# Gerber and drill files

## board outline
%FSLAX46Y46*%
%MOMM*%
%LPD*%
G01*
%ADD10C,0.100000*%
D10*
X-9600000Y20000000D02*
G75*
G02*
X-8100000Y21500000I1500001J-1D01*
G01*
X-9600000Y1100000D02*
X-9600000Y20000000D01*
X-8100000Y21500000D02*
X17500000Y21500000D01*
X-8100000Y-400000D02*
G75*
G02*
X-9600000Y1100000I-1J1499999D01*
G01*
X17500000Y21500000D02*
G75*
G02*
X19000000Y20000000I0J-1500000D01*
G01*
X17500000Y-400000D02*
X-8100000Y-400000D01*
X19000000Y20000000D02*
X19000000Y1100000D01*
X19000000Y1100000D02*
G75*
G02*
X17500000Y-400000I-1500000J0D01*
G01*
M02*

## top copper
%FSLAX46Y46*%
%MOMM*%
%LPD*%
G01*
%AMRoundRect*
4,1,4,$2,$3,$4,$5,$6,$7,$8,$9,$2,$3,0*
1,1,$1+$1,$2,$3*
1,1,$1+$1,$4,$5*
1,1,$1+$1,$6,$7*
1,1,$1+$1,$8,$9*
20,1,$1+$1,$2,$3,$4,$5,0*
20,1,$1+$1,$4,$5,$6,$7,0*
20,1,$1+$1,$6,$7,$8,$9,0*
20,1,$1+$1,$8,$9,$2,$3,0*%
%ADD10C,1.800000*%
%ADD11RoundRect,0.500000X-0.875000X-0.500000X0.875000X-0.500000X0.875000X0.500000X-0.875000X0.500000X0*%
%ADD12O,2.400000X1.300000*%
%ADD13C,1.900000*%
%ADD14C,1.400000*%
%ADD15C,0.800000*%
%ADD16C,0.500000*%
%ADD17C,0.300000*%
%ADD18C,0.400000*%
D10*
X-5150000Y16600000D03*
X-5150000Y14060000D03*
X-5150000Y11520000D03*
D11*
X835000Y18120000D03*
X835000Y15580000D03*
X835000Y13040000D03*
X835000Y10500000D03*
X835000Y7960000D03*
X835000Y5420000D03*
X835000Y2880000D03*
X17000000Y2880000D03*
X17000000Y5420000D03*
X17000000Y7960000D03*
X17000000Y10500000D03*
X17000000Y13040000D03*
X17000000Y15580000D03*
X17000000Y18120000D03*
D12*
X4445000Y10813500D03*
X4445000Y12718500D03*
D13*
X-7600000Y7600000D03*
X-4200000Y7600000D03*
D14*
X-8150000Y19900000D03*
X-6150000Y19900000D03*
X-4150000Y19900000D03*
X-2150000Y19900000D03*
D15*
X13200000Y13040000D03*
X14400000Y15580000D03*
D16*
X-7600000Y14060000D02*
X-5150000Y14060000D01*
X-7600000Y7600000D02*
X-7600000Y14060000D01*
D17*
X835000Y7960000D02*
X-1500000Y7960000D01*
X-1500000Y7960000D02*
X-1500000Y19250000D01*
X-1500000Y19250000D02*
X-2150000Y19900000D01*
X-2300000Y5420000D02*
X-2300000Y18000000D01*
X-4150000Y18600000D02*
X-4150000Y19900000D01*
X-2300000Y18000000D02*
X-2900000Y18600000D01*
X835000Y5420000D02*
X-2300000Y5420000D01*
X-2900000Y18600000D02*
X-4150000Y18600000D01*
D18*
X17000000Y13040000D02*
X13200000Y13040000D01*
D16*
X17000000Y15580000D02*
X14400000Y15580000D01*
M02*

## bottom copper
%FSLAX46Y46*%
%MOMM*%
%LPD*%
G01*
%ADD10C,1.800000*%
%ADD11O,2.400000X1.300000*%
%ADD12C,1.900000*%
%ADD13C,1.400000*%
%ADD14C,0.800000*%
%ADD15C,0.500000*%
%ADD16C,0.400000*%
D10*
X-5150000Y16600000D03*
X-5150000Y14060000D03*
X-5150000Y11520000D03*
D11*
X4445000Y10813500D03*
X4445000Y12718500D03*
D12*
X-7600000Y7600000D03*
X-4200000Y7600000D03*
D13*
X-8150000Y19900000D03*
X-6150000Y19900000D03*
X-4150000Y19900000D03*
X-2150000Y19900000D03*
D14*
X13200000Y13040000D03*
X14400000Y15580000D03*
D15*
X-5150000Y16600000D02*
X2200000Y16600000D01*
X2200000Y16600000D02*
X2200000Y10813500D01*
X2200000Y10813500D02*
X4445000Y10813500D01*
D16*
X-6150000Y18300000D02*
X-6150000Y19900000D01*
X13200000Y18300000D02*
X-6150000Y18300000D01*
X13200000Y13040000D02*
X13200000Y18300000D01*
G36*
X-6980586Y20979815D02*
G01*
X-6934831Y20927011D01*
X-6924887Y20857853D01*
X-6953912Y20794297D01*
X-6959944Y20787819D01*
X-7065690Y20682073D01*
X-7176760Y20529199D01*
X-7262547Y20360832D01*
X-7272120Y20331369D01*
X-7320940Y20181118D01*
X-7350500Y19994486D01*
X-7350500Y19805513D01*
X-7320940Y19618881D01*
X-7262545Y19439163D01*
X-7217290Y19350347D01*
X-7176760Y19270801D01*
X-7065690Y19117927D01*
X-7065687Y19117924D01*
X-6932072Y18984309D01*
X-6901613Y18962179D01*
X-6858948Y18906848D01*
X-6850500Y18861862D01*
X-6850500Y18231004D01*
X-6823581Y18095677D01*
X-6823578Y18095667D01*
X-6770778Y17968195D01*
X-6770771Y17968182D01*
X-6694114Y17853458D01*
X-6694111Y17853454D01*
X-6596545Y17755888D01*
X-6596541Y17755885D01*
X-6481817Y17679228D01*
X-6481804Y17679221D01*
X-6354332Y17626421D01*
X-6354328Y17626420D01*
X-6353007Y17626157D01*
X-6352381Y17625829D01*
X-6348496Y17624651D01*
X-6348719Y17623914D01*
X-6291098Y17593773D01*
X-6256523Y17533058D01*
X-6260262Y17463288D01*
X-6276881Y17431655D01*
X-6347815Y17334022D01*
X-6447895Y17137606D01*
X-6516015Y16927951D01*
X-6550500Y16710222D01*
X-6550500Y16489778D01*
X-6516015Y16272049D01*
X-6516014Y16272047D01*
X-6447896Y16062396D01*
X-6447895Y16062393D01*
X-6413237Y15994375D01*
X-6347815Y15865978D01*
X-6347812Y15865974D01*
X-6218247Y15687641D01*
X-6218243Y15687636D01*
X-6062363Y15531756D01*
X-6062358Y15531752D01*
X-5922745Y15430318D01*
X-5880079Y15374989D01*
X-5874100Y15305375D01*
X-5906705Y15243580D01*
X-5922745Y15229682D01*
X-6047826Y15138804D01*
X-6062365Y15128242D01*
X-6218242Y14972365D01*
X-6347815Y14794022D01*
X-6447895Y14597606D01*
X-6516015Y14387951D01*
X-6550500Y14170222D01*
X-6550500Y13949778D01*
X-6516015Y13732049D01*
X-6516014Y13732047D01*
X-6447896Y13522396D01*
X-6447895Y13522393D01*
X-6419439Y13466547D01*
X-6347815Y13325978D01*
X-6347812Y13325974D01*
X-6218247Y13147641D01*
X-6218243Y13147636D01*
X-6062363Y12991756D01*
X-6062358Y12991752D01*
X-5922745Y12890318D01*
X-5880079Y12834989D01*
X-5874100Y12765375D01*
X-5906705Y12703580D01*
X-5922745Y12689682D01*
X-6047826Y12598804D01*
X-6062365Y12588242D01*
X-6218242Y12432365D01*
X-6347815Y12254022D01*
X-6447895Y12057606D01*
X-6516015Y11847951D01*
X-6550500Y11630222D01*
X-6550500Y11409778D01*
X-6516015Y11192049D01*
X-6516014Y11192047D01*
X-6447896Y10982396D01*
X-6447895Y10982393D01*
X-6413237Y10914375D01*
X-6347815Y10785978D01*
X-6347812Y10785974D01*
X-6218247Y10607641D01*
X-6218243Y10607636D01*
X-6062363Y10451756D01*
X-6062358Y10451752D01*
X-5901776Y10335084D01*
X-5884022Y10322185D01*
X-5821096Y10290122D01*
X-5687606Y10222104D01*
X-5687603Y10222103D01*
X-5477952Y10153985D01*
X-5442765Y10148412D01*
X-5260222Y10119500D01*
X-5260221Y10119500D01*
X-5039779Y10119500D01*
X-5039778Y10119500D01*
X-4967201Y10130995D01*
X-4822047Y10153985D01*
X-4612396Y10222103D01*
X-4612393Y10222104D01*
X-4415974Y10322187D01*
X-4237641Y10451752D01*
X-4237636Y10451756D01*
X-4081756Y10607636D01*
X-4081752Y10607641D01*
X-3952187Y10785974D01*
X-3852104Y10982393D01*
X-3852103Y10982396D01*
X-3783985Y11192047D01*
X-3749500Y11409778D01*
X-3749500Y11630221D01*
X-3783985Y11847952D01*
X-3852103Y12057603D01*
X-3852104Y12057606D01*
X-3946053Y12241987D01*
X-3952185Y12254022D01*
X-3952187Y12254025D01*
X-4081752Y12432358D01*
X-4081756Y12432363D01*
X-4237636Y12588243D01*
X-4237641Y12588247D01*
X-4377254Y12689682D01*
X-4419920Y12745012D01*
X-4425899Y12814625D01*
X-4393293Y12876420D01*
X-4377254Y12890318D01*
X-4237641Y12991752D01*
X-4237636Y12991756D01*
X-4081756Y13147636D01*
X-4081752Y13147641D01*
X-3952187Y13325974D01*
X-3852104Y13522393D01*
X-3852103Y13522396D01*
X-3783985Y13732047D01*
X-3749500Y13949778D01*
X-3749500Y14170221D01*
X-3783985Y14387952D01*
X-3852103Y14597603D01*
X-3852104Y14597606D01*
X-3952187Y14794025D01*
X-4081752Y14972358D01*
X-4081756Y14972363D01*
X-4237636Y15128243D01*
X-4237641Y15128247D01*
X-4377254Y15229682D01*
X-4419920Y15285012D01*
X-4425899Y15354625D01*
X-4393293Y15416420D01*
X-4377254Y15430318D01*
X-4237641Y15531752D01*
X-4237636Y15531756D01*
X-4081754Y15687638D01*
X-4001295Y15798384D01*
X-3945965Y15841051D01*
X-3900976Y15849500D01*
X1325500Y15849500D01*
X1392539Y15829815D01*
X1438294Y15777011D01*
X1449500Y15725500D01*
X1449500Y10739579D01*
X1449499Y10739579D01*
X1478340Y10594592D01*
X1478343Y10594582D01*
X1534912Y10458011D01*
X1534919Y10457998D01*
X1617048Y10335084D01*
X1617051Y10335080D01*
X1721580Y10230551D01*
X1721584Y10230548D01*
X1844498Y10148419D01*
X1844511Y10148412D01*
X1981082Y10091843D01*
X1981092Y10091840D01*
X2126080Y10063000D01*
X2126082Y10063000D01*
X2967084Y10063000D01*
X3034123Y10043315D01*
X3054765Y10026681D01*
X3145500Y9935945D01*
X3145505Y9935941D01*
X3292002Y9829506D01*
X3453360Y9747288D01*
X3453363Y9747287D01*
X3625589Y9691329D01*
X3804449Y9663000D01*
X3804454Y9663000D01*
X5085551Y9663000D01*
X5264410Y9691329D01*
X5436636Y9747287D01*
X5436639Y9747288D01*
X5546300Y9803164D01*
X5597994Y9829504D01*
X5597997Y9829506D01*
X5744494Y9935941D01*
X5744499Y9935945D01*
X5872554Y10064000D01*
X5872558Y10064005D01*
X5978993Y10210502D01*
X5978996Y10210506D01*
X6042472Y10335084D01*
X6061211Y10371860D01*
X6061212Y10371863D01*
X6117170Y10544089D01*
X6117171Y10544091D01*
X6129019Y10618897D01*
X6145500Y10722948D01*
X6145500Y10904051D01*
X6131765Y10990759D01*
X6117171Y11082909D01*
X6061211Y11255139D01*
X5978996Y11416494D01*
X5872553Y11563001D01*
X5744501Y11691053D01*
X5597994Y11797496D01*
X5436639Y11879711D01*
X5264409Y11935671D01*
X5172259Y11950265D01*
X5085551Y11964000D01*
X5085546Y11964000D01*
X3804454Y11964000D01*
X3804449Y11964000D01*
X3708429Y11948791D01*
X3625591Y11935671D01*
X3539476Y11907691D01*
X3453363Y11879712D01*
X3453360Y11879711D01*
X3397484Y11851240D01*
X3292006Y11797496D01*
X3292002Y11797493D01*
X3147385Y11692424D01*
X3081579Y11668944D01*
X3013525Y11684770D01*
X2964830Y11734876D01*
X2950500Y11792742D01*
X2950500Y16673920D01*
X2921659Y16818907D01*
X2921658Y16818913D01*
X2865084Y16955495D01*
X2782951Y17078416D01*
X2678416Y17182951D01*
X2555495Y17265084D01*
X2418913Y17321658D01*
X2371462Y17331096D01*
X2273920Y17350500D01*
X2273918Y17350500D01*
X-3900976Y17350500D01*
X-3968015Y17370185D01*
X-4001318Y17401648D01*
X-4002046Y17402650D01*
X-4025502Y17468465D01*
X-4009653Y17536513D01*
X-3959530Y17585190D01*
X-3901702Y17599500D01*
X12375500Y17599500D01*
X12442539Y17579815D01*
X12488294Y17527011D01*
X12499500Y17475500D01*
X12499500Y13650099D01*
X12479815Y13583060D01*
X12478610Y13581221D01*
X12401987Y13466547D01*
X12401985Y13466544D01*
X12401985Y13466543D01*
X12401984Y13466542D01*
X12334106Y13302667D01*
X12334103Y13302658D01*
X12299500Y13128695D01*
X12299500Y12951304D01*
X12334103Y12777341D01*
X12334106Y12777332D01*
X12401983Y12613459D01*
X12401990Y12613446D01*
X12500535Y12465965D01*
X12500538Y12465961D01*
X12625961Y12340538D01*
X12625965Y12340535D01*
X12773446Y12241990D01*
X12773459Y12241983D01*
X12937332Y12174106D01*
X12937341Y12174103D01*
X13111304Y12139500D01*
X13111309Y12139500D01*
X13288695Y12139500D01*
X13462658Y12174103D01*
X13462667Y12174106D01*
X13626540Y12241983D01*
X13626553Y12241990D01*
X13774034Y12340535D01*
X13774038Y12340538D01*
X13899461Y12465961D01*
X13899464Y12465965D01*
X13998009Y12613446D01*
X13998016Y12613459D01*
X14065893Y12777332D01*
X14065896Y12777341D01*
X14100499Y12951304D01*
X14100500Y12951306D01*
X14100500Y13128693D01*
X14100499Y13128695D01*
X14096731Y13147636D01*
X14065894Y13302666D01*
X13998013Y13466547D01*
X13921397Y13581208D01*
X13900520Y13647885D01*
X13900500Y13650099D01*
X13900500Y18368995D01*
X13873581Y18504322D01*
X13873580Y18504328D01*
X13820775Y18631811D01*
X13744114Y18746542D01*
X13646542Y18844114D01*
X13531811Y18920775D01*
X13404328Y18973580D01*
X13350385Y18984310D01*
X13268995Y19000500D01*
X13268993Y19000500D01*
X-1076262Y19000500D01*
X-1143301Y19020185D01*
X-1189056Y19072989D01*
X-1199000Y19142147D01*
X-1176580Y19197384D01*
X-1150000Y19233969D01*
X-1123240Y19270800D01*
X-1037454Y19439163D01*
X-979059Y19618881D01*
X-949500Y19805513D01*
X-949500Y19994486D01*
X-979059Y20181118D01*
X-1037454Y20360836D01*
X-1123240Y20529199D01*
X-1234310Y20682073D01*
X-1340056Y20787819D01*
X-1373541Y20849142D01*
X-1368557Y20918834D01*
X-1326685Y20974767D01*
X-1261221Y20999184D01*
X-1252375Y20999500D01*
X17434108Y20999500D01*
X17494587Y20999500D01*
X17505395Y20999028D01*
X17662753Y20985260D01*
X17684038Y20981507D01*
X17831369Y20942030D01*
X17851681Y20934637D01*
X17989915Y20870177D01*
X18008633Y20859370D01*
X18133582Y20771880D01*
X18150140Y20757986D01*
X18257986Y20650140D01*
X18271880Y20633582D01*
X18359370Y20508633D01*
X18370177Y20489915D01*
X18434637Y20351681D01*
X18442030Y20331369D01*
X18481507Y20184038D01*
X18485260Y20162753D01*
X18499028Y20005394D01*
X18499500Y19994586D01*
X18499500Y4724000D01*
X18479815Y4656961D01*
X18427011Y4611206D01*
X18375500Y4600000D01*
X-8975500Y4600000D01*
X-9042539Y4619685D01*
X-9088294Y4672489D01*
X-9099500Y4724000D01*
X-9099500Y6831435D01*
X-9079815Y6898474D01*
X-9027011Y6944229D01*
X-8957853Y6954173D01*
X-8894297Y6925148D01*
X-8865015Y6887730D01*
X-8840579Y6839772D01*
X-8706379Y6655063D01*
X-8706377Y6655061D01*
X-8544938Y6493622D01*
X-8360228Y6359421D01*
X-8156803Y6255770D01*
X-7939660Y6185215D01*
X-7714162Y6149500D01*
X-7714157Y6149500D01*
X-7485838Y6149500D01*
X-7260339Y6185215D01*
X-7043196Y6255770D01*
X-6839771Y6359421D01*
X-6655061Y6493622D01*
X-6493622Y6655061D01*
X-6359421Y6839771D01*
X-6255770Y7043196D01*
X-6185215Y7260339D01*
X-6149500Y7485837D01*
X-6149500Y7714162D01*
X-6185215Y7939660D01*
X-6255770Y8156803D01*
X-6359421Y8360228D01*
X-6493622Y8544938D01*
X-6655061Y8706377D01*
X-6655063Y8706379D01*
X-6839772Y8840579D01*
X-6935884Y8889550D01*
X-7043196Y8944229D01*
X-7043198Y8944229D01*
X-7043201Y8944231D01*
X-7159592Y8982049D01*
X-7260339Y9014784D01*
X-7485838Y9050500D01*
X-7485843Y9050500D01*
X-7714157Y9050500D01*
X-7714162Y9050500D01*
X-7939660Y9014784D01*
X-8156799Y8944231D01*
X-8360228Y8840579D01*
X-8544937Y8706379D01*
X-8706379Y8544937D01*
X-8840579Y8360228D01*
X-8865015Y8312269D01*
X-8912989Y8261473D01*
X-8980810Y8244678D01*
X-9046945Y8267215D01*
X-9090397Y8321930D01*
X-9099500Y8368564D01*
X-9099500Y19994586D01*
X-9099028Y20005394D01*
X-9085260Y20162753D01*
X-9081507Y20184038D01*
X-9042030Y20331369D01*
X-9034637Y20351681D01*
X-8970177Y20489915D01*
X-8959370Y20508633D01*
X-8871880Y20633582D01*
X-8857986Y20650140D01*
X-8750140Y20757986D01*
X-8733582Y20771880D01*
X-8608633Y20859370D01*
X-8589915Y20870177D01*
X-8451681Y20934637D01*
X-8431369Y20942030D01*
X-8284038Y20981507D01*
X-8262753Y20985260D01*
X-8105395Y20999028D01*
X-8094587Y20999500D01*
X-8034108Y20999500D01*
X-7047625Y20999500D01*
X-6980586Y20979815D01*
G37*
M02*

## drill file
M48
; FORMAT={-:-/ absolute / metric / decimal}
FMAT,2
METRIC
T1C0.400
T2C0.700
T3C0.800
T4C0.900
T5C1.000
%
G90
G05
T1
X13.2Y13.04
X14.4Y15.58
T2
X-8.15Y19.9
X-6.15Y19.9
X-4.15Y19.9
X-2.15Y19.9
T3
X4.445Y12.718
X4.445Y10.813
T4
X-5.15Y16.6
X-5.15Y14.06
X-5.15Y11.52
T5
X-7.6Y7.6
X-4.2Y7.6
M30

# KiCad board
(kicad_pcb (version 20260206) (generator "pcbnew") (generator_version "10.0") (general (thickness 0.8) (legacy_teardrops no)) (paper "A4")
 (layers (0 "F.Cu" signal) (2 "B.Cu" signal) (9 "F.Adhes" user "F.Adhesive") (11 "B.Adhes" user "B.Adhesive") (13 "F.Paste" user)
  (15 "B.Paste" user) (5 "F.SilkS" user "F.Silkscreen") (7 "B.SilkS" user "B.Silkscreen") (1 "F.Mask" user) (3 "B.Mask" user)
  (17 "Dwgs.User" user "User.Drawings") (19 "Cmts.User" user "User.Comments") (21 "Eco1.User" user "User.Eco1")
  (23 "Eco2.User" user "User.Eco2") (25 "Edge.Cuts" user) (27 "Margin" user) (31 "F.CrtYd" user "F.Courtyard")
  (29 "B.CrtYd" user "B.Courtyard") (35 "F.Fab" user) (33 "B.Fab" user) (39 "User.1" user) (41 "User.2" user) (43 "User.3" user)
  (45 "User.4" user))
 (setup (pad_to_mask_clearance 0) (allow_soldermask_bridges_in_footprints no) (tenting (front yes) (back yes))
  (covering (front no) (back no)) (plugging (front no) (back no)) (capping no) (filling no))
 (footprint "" (layer "F.Cu") (at 0 0)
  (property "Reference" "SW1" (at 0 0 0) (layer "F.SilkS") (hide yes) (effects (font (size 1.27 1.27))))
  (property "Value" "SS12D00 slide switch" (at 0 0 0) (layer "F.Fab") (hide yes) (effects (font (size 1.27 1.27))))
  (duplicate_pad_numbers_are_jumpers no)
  (pad "1" thru_hole circle (at -5.15 -16.6) (size 1.8 1.8) (drill 0.9) (layers "*.Cu" "*.Mask") (remove_unused_layers no)
   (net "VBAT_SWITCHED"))
  (pad "2" thru_hole circle (at -5.15 -14.06) (size 1.8 1.8) (drill 0.9) (layers "*.Cu" "*.Mask") (remove_unused_layers no) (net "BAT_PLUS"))
  (pad "3" thru_hole circle (at -5.15 -11.52) (size 1.8 1.8) (drill 0.9) (layers "*.Cu" "*.Mask") (remove_unused_layers no)))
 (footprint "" (layer "F.Cu") (at 0 0)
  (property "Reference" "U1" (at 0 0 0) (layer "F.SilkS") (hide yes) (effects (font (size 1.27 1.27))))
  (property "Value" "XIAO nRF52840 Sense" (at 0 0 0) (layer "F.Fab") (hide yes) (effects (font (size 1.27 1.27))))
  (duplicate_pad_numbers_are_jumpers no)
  (pad "1" smd roundrect (at 0.835 -18.12) (size 2.75 2) (layers "F.Cu" "F.Mask" "F.Paste") (roundrect_rratio 0.25)
   (thermal_bridge_angle 45))
  (pad "2" smd roundrect (at 0.835 -15.58) (size 2.75 2) (layers "F.Cu" "F.Mask" "F.Paste") (roundrect_rratio 0.25)
   (thermal_bridge_angle 45))
  (pad "3" smd roundrect (at 0.835 -13.04) (size 2.75 2) (layers "F.Cu" "F.Mask" "F.Paste") (roundrect_rratio 0.25)
   (thermal_bridge_angle 45))
  (pad "4" smd roundrect (at 0.835 -10.5) (size 2.75 2) (layers "F.Cu" "F.Mask" "F.Paste") (roundrect_rratio 0.25) (thermal_bridge_angle 45))
  (pad "5" smd roundrect (at 0.835 -7.96) (size 2.75 2) (layers "F.Cu" "F.Mask" "F.Paste") (roundrect_rratio 0.25) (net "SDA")
   (thermal_bridge_angle 45))
  (pad "6" smd roundrect (at 0.835 -5.42) (size 2.75 2) (layers "F.Cu" "F.Mask" "F.Paste") (roundrect_rratio 0.25) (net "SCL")
   (thermal_bridge_angle 45))
  (pad "7" smd roundrect (at 0.835 -2.88) (size 2.75 2) (layers "F.Cu" "F.Mask" "F.Paste") (roundrect_rratio 0.25) (thermal_bridge_angle 45))
  (pad "8" smd roundrect (at 17 -2.88) (size 2.75 2) (layers "F.Cu" "F.Mask" "F.Paste") (roundrect_rratio 0.25) (thermal_bridge_angle 45))
  (pad "9" smd roundrect (at 17 -5.42) (size 2.75 2) (layers "F.Cu" "F.Mask" "F.Paste") (roundrect_rratio 0.25) (thermal_bridge_angle 45))
  (pad "10" smd roundrect (at 17 -7.96) (size 2.75 2) (layers "F.Cu" "F.Mask" "F.Paste") (roundrect_rratio 0.25) (thermal_bridge_angle 45))
  (pad "11" smd roundrect (at 17 -10.5) (size 2.75 2) (layers "F.Cu" "F.Mask" "F.Paste") (roundrect_rratio 0.25) (thermal_bridge_angle 45))
  (pad "12" smd roundrect (at 17 -13.04) (size 2.75 2) (layers "F.Cu" "F.Mask" "F.Paste") (roundrect_rratio 0.25) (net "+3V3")
   (thermal_bridge_angle 45))
  (pad "13" smd roundrect (at 17 -15.58) (size 2.75 2) (layers "F.Cu" "F.Mask" "F.Paste") (roundrect_rratio 0.25) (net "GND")
   (thermal_bridge_angle 45))
  (pad "14" smd roundrect (at 17 -18.12) (size 2.75 2) (layers "F.Cu" "F.Mask" "F.Paste") (roundrect_rratio 0.25) (thermal_bridge_angle 45))
  (pad "19" thru_hole oval (at 4.445 -10.8135) (size 2.4 1.3) (drill 0.8) (layers "*.Cu" "*.Mask") (remove_unused_layers no)
   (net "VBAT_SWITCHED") (thermal_bridge_angle 45))
  (pad "20" thru_hole oval (at 4.445 -12.7185) (size 2.4 1.3) (drill 0.8) (layers "*.Cu" "*.Mask") (remove_unused_layers no) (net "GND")
   (thermal_bridge_angle 45)))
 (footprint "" (layer "F.Cu") (at 0 0)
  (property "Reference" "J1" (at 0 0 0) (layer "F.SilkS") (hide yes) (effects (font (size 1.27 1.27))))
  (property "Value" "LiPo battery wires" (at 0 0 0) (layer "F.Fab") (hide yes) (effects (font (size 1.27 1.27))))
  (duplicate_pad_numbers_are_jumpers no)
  (pad "1" thru_hole circle (at -7.6 -7.6) (size 1.9 1.9) (drill 1) (layers "*.Cu" "*.Mask") (remove_unused_layers no) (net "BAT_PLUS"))
  (pad "2" thru_hole circle (at -4.2 -7.6) (size 1.9 1.9) (drill 1) (layers "*.Cu" "*.Mask") (remove_unused_layers no) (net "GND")))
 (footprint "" (layer "F.Cu") (at 0 0)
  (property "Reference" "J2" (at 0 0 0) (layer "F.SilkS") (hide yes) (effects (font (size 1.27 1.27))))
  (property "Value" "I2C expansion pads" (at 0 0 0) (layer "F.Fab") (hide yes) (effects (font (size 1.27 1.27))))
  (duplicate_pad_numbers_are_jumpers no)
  (pad "1" thru_hole circle (at -8.15 -19.9) (size 1.4 1.4) (drill 0.7) (layers "*.Cu" "*.Mask") (remove_unused_layers no) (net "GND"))
  (pad "2" thru_hole circle (at -6.15 -19.9) (size 1.4 1.4) (drill 0.7) (layers "*.Cu" "*.Mask") (remove_unused_layers no) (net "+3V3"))
  (pad "3" thru_hole circle (at -4.15 -19.9) (size 1.4 1.4) (drill 0.7) (layers "*.Cu" "*.Mask") (remove_unused_layers no) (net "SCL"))
  (pad "4" thru_hole circle (at -2.15 -19.9) (size 1.4 1.4) (drill 0.7) (layers "*.Cu" "*.Mask") (remove_unused_layers no) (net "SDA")))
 (gr_arc (start -9.6 -20) (mid -9.16066 -21.06066) (end -8.1 -21.5) (stroke (width 0.1) (type default)) (layer "Edge.Cuts"))
 (gr_line (start -9.6 -1.1) (end -9.6 -20) (stroke (width 0.1) (type default)) (layer "Edge.Cuts"))
 (gr_line (start -8.1 -21.5) (end 17.5 -21.5) (stroke (width 0.1) (type default)) (layer "Edge.Cuts"))
 (gr_arc (start -8.1 0.4) (mid -9.16066 -0.039339) (end -9.6 -1.1) (stroke (width 0.1) (type default)) (layer "Edge.Cuts"))
 (gr_arc (start 17.5 -21.5) (mid 18.56066 -21.06066) (end 19 -20) (stroke (width 0.1) (type default)) (layer "Edge.Cuts"))
 (gr_line (start 17.5 0.4) (end -8.1 0.4) (stroke (width 0.1) (type default)) (layer "Edge.Cuts"))
 (gr_line (start 19 -20) (end 19 -1.1) (stroke (width 0.1) (type default)) (layer "Edge.Cuts"))
 (gr_arc (start 19 -1.1) (mid 18.56066 -0.039339) (end 17.5 0.4) (stroke (width 0.1) (type default)) (layer "Edge.Cuts"))
 (segment (start -5.15 -16.6) (end 2.2 -16.6) (width 0.5) (layer "B.Cu") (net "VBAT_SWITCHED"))
 (segment (start 2.2 -16.6) (end 2.2 -10.8135) (width 0.5) (layer "B.Cu") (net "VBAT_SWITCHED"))
 (segment (start 2.2 -10.8135) (end 4.445 -10.8135) (width 0.5) (layer "B.Cu") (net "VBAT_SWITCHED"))
 (segment (start -7.6 -14.06) (end -5.15 -14.06) (width 0.5) (layer "F.Cu") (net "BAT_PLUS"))
 (segment (start -7.6 -7.6) (end -7.6 -14.06) (width 0.5) (layer "F.Cu") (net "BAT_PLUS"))
 (segment (start 0.835 -7.96) (end -1.5 -7.96) (width 0.3) (layer "F.Cu") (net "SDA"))
 (segment (start -1.5 -7.96) (end -1.5 -19.25) (width 0.3) (layer "F.Cu") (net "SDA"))
 (segment (start -1.5 -19.25) (end -2.15 -19.9) (width 0.3) (layer "F.Cu") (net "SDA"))
 (segment (start -2.3 -5.42) (end -2.3 -18) (width 0.3) (layer "F.Cu") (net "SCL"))
 (segment (start -4.15 -18.6) (end -4.15 -19.9) (width 0.3) (layer "F.Cu") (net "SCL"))
 (segment (start -2.3 -18) (end -2.9 -18.6) (width 0.3) (layer "F.Cu") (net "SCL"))
 (segment (start 0.835 -5.42) (end -2.3 -5.42) (width 0.3) (layer "F.Cu") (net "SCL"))
 (segment (start -2.9 -18.6) (end -4.15 -18.6) (width 0.3) (layer "F.Cu") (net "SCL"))
 (segment (start 17 -13.04) (end 13.2 -13.04) (width 0.4) (layer "F.Cu") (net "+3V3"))
 (via (at 13.2 -13.04) (size 0.8) (drill 0.4) (layers "F.Cu" "B.Cu") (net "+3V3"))
 (segment (start -6.15 -18.3) (end -6.15 -19.9) (width 0.4) (layer "B.Cu") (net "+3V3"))
 (segment (start 13.2 -18.3) (end -6.15 -18.3) (width 0.4) (layer "B.Cu") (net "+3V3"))
 (segment (start 13.2 -13.04) (end 13.2 -18.3) (width 0.4) (layer "B.Cu") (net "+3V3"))
 (segment (start 17 -15.58) (end 14.4 -15.58) (width 0.5) (layer "F.Cu") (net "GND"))
 (via (at 14.4 -15.58) (size 0.8) (drill 0.4) (layers "F.Cu" "B.Cu") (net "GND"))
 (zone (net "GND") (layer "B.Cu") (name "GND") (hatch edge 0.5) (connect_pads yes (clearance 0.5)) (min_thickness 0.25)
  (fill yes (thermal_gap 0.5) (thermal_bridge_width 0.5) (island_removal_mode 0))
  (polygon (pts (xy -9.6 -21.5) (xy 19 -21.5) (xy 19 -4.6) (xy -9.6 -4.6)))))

